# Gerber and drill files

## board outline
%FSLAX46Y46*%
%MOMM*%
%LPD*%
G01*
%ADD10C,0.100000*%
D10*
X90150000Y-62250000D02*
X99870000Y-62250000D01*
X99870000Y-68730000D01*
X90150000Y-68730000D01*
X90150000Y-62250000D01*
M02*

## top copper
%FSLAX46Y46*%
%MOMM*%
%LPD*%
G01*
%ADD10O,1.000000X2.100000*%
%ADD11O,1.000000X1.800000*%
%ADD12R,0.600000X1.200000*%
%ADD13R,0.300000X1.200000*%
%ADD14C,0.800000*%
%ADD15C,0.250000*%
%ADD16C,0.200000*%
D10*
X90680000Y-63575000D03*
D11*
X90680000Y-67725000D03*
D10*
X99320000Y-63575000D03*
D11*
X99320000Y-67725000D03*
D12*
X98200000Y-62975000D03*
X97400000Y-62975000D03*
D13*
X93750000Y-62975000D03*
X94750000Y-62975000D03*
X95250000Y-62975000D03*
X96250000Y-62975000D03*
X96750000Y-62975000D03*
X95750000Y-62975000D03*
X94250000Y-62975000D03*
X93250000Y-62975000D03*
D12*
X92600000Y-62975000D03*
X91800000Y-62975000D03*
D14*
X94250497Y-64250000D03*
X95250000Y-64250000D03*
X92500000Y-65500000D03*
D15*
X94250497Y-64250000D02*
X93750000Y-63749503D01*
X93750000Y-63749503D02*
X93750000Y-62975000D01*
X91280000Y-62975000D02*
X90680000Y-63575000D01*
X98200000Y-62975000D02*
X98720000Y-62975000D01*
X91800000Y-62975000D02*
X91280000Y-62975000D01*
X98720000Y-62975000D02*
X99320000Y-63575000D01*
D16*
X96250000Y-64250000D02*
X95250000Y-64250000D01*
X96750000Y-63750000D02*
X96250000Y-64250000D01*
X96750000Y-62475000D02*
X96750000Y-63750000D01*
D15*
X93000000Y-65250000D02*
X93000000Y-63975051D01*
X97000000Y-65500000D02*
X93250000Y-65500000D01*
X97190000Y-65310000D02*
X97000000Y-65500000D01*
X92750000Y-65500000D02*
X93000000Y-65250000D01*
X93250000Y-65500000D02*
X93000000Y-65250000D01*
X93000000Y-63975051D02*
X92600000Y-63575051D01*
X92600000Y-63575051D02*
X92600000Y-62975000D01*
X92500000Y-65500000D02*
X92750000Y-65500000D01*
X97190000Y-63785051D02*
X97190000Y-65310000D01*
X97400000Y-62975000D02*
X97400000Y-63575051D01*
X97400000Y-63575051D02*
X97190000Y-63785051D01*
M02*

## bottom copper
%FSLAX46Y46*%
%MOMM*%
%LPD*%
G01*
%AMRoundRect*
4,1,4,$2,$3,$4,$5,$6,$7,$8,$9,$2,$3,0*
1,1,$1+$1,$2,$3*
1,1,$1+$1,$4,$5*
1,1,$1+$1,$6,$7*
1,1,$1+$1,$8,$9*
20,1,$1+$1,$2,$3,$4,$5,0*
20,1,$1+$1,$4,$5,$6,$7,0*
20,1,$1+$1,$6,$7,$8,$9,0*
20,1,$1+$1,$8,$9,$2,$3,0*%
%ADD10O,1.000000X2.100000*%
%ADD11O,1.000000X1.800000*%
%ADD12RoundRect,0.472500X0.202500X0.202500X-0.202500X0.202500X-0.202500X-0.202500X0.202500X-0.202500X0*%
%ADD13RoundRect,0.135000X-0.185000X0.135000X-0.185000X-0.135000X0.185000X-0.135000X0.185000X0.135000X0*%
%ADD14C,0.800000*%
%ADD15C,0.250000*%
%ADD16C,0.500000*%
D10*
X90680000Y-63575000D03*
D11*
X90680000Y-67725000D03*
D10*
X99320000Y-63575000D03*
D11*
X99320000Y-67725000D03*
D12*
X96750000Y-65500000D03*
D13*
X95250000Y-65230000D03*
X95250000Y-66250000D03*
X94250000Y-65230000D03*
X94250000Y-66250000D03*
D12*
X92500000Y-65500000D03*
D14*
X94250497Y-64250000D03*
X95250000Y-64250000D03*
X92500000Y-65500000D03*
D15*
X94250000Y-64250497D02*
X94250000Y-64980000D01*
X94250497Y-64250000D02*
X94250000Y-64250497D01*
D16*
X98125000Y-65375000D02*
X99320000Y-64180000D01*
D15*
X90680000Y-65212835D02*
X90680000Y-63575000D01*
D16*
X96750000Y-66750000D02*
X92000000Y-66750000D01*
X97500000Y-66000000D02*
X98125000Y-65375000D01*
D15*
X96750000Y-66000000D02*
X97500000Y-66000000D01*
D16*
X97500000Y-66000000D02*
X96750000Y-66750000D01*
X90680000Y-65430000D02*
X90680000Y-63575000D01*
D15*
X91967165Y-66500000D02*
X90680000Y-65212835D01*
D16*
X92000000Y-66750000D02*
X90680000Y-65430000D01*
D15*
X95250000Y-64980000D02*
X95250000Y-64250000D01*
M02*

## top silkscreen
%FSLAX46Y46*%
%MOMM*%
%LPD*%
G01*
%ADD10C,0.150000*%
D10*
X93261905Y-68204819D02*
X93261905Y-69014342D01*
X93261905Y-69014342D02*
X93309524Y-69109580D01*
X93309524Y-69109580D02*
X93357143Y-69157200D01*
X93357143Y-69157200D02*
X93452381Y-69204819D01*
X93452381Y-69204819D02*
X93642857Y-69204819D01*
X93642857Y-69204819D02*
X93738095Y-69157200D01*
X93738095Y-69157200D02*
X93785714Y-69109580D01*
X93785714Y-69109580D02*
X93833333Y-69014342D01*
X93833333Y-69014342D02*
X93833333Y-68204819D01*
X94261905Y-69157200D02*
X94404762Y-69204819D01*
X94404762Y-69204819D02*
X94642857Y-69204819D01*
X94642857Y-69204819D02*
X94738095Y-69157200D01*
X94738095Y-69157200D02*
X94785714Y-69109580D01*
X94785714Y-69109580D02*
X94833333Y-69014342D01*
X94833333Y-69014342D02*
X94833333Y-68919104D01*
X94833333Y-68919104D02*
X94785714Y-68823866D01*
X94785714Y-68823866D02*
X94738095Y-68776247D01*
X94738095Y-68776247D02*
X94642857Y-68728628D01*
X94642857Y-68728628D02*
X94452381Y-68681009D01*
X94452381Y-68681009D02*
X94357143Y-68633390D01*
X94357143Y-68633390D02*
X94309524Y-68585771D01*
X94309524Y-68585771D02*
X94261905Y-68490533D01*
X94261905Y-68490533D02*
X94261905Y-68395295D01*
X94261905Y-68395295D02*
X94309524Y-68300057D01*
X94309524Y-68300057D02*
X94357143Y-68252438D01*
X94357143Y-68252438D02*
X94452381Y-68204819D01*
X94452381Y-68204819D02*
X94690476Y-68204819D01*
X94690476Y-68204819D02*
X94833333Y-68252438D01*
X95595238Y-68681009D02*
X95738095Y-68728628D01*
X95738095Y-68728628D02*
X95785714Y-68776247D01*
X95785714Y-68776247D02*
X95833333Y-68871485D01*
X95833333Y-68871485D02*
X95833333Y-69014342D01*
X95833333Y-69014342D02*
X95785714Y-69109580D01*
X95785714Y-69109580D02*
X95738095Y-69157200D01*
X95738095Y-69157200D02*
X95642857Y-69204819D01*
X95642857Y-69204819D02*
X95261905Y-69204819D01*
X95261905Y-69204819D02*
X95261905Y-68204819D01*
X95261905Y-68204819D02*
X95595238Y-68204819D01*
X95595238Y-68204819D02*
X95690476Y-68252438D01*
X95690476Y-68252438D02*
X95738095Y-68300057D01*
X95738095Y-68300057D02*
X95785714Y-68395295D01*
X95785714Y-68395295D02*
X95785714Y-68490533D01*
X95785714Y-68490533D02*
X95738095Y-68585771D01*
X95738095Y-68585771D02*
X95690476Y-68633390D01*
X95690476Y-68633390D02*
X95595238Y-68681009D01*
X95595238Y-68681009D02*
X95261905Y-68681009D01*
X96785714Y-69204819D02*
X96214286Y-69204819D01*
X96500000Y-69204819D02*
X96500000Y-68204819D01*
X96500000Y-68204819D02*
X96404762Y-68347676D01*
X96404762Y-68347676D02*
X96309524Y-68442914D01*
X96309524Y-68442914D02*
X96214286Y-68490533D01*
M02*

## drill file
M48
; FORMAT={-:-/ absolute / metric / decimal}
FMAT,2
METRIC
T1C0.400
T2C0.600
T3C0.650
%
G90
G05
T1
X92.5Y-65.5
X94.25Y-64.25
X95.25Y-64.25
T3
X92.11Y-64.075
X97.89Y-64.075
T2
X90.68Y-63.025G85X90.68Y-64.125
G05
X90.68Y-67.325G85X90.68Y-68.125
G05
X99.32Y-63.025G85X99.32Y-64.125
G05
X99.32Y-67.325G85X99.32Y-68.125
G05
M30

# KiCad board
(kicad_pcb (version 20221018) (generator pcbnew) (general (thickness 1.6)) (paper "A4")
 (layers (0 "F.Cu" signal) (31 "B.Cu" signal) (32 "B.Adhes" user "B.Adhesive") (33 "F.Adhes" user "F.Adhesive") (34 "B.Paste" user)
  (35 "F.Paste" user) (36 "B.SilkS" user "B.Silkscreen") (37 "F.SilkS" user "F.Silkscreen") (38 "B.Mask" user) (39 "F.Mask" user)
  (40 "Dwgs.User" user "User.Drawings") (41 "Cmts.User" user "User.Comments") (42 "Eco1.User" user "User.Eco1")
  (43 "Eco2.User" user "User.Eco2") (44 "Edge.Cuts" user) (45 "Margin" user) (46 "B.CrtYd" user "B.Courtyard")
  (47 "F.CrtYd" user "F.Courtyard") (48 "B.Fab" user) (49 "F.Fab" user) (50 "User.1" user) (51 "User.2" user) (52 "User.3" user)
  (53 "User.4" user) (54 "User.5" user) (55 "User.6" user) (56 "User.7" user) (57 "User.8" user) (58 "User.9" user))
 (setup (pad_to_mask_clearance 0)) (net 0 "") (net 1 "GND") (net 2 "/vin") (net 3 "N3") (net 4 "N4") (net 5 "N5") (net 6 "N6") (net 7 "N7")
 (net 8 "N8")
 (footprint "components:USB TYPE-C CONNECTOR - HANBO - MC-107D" (layer "F.Cu") (at 95 70.375)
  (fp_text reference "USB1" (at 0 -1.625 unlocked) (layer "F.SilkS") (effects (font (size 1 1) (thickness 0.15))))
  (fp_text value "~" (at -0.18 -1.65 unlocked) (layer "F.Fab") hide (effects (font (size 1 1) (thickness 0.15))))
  (pad "" thru_hole oval (at -4.32 -6.8) (size 1 2.1) (drill oval 0.6 1.7) (layers "*.Cu" "*.Mask") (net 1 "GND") (thermal_bridge_angle 45))
  (pad "" thru_hole oval (at -4.32 -2.65) (size 1 1.8) (drill oval 0.6 1.4) (layers "*.Cu" "*.Mask") (thermal_bridge_angle 45))
  (pad "" np_thru_hole circle (at -2.89 -6.3) (size 0.65 0.65) (drill 0.65) (layers "F&B.Cu" "*.Mask"))
  (pad "" np_thru_hole circle (at 2.89 -6.3) (size 0.65 0.65) (drill 0.65) (layers "F&B.Cu" "*.Mask"))
  (pad "" thru_hole oval (at 4.32 -6.8) (size 1 2.1) (drill oval 0.6 1.7) (layers "*.Cu" "*.Mask") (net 1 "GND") (thermal_bridge_angle 45))
  (pad "" thru_hole oval (at 4.32 -2.65) (size 1 1.8) (drill oval 0.6 1.4) (layers "*.Cu" "*.Mask") (thermal_bridge_angle 45))
  (pad "A1" smd rect (at 3.2 -7.4) (size 0.6 1.2) (layers "F.Cu" "F.Paste" "F.Mask") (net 1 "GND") (thermal_bridge_angle 45))
  (pad "A4" smd rect (at 2.4 -7.4) (size 0.6 1.2) (layers "F.Cu" "F.Paste" "F.Mask") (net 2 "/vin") (thermal_bridge_angle 45))
  (pad "A5" smd rect (at -1.25 -7.4) (size 0.3 1.2) (layers "F.Cu" "F.Paste" "F.Mask") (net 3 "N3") (thermal_bridge_angle 45))
  (pad "A6" smd rect (at -0.25 -7.4) (size 0.3 1.2) (layers "F.Cu" "F.Paste" "F.Mask") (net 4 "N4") (thermal_bridge_angle 45))
  (pad "A7" smd rect (at 0.25 -7.4) (size 0.3 1.2) (layers "F.Cu" "F.Paste" "F.Mask") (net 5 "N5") (thermal_bridge_angle 45))
  (pad "A8" smd rect (at 1.25 -7.4) (size 0.3 1.2) (layers "F.Cu" "F.Paste" "F.Mask") (thermal_bridge_angle 45))
  (pad "B5" smd rect (at 1.75 -7.4) (size 0.3 1.2) (layers "F.Cu" "F.Paste" "F.Mask") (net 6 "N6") (thermal_bridge_angle 45))
  (pad "B6" smd rect (at 0.75 -7.4) (size 0.3 1.2) (layers "F.Cu" "F.Paste" "F.Mask") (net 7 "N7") (thermal_bridge_angle 45))
  (pad "B7" smd rect (at -0.75 -7.4) (size 0.3 1.2) (layers "F.Cu" "F.Paste" "F.Mask") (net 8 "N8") (thermal_bridge_angle 45))
  (pad "B8" smd rect (at -1.75 -7.4) (size 0.3 1.2) (layers "F.Cu" "F.Paste" "F.Mask") (thermal_bridge_angle 45))
  (pad "B9" smd rect (at -2.4 -7.4) (size 0.6 1.2) (layers "F.Cu" "F.Paste" "F.Mask") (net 2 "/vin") (thermal_bridge_angle 45))
  (pad "B12" smd rect (at -3.2 -7.4) (size 0.6 1.2) (layers "F.Cu" "F.Paste" "F.Mask") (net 1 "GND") (thermal_bridge_angle 45)))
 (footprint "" (layer "B.Cu") (at 96.75 65.5 180)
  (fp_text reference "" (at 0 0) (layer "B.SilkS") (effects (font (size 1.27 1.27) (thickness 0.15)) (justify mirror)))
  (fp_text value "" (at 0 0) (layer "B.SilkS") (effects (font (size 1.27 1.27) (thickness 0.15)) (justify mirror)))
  (pad "1" smd roundrect (at 0 0 180) (size 1.35 1.35) (layers "B.Cu" "B.Paste" "B.Mask") (roundrect_rratio 0.35) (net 1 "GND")))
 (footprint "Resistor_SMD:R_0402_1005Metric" (layer "B.Cu") (at 95.25 65.74 -90)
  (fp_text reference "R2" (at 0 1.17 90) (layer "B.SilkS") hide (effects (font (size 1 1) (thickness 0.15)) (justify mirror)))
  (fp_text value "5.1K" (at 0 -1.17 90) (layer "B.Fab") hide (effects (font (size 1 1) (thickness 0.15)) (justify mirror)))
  (pad "1" smd roundrect (at -0.51 0 270) (size 0.54 0.64) (layers "B.Cu" "B.Paste" "B.Mask") (roundrect_rratio 0.25) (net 6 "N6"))
  (pad "2" smd roundrect (at 0.51 0 270) (size 0.54 0.64) (layers "B.Cu" "B.Paste" "B.Mask") (roundrect_rratio 0.25) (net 1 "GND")))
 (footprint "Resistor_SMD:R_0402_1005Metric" (layer "B.Cu") (at 94.25 65.74 -90)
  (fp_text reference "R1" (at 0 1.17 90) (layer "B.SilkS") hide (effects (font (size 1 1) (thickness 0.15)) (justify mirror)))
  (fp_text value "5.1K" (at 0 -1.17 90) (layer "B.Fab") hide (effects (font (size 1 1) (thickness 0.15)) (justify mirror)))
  (pad "1" smd roundrect (at -0.51 0 270) (size 0.54 0.64) (layers "B.Cu" "B.Paste" "B.Mask") (roundrect_rratio 0.25) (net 3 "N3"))
  (pad "2" smd roundrect (at 0.51 0 270) (size 0.54 0.64) (layers "B.Cu" "B.Paste" "B.Mask") (roundrect_rratio 0.25) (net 1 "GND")))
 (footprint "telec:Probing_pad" (layer "B.Cu") (at 92.5 65.5 180)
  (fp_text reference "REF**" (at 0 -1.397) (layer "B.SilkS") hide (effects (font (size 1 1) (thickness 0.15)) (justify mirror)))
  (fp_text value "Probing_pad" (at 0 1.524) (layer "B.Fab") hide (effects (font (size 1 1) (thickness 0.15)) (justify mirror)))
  (pad "1" smd roundrect (at 0 0 180) (size 1.35 1.35) (layers "B.Cu" "B.Paste" "B.Mask") (roundrect_rratio 0.35) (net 2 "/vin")))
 (gr_rect (start 90.15 62.25) (end 99.87 68.73) (stroke (width 0.1) (type default)) (fill none) (layer "Edge.Cuts"))
 (segment (start 94.250497 64.25) (end 93.75 63.749503) (width 0.25) (layer "F.Cu") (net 3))
 (segment (start 93.75 63.749503) (end 93.75 62.975) (width 0.25) (layer "F.Cu") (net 3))
 (via (at 94.250497 64.25) (size 0.8) (drill 0.4) (layers "F.Cu" "B.Cu") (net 3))
 (segment (start 94.25 64.250497) (end 94.25 64.98) (width 0.25) (layer "B.Cu") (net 3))
 (segment (start 94.250497 64.25) (end 94.25 64.250497) (width 0.25) (layer "B.Cu") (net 3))
 (segment (start 91.28 62.975) (end 90.68 63.575) (width 0.25) (layer "F.Cu") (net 1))
 (segment (start 98.2 62.975) (end 98.72 62.975) (width 0.25) (layer "F.Cu") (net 1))
 (segment (start 91.8 62.975) (end 91.28 62.975) (width 0.25) (layer "F.Cu") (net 1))
 (segment (start 98.72 62.975) (end 99.32 63.575) (width 0.25) (layer "F.Cu") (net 1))
 (segment (start 98.125 65.375) (end 99.32 64.18) (width 0.5) (layer "B.Cu") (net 1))
 (segment (start 90.68 65.212835) (end 90.68 63.575) (width 0.25) (layer "B.Cu") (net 1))
 (segment (start 96.75 66.75) (end 92 66.75) (width 0.5) (layer "B.Cu") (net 1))
 (segment (start 97.5 66) (end 98.125 65.375) (width 0.5) (layer "B.Cu") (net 1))
 (segment (start 96.75 66) (end 97.5 66) (width 0.25) (layer "B.Cu") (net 1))
 (segment (start 97.5 66) (end 96.75 66.75) (width 0.5) (layer "B.Cu") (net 1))
 (segment (start 90.68 65.43) (end 90.68 63.575) (width 0.5) (layer "B.Cu") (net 1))
 (segment (start 91.967165 66.5) (end 90.68 65.212835) (width 0.25) (layer "B.Cu") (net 1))
 (segment (start 92 66.75) (end 90.68 65.43) (width 0.5) (layer "B.Cu") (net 1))
 (segment (start 96.25 64.25) (end 95.25 64.25) (width 0.2) (layer "F.Cu") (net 6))
 (segment (start 96.75 63.75) (end 96.25 64.25) (width 0.2) (layer "F.Cu") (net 6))
 (segment (start 96.75 62.475) (end 96.75 63.75) (width 0.2) (layer "F.Cu") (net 6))
 (via (at 95.25 64.25) (size 0.8) (drill 0.4) (layers "F.Cu" "B.Cu") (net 6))
 (segment (start 95.25 64.98) (end 95.25 64.25) (width 0.25) (layer "B.Cu") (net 6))
 (segment (start 93 65.25) (end 93 63.975051) (width 0.25) (layer "F.Cu") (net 2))
 (segment (start 97 65.5) (end 93.25 65.5) (width 0.25) (layer "F.Cu") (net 2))
 (segment (start 97.19 65.31) (end 97 65.5) (width 0.25) (layer "F.Cu") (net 2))
 (segment (start 92.75 65.5) (end 93 65.25) (width 0.25) (layer "F.Cu") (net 2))
 (segment (start 93.25 65.5) (end 93 65.25) (width 0.25) (layer "F.Cu") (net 2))
 (segment (start 93 63.975051) (end 92.6 63.575051) (width 0.25) (layer "F.Cu") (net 2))
 (segment (start 92.6 63.575051) (end 92.6 62.975) (width 0.25) (layer "F.Cu") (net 2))
 (segment (start 92.5 65.5) (end 92.75 65.5) (width 0.25) (layer "F.Cu") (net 2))
 (segment (start 97.19 63.785051) (end 97.19 65.31) (width 0.25) (layer "F.Cu") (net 2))
 (segment (start 97.4 62.975) (end 97.4 63.575051) (width 0.25) (layer "F.Cu") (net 2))
 (segment (start 97.4 63.575051) (end 97.19 63.785051) (width 0.25) (layer "F.Cu") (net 2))
 (via (at 92.5 65.5) (size 0.8) (drill 0.4) (layers "F.Cu" "B.Cu") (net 2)))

